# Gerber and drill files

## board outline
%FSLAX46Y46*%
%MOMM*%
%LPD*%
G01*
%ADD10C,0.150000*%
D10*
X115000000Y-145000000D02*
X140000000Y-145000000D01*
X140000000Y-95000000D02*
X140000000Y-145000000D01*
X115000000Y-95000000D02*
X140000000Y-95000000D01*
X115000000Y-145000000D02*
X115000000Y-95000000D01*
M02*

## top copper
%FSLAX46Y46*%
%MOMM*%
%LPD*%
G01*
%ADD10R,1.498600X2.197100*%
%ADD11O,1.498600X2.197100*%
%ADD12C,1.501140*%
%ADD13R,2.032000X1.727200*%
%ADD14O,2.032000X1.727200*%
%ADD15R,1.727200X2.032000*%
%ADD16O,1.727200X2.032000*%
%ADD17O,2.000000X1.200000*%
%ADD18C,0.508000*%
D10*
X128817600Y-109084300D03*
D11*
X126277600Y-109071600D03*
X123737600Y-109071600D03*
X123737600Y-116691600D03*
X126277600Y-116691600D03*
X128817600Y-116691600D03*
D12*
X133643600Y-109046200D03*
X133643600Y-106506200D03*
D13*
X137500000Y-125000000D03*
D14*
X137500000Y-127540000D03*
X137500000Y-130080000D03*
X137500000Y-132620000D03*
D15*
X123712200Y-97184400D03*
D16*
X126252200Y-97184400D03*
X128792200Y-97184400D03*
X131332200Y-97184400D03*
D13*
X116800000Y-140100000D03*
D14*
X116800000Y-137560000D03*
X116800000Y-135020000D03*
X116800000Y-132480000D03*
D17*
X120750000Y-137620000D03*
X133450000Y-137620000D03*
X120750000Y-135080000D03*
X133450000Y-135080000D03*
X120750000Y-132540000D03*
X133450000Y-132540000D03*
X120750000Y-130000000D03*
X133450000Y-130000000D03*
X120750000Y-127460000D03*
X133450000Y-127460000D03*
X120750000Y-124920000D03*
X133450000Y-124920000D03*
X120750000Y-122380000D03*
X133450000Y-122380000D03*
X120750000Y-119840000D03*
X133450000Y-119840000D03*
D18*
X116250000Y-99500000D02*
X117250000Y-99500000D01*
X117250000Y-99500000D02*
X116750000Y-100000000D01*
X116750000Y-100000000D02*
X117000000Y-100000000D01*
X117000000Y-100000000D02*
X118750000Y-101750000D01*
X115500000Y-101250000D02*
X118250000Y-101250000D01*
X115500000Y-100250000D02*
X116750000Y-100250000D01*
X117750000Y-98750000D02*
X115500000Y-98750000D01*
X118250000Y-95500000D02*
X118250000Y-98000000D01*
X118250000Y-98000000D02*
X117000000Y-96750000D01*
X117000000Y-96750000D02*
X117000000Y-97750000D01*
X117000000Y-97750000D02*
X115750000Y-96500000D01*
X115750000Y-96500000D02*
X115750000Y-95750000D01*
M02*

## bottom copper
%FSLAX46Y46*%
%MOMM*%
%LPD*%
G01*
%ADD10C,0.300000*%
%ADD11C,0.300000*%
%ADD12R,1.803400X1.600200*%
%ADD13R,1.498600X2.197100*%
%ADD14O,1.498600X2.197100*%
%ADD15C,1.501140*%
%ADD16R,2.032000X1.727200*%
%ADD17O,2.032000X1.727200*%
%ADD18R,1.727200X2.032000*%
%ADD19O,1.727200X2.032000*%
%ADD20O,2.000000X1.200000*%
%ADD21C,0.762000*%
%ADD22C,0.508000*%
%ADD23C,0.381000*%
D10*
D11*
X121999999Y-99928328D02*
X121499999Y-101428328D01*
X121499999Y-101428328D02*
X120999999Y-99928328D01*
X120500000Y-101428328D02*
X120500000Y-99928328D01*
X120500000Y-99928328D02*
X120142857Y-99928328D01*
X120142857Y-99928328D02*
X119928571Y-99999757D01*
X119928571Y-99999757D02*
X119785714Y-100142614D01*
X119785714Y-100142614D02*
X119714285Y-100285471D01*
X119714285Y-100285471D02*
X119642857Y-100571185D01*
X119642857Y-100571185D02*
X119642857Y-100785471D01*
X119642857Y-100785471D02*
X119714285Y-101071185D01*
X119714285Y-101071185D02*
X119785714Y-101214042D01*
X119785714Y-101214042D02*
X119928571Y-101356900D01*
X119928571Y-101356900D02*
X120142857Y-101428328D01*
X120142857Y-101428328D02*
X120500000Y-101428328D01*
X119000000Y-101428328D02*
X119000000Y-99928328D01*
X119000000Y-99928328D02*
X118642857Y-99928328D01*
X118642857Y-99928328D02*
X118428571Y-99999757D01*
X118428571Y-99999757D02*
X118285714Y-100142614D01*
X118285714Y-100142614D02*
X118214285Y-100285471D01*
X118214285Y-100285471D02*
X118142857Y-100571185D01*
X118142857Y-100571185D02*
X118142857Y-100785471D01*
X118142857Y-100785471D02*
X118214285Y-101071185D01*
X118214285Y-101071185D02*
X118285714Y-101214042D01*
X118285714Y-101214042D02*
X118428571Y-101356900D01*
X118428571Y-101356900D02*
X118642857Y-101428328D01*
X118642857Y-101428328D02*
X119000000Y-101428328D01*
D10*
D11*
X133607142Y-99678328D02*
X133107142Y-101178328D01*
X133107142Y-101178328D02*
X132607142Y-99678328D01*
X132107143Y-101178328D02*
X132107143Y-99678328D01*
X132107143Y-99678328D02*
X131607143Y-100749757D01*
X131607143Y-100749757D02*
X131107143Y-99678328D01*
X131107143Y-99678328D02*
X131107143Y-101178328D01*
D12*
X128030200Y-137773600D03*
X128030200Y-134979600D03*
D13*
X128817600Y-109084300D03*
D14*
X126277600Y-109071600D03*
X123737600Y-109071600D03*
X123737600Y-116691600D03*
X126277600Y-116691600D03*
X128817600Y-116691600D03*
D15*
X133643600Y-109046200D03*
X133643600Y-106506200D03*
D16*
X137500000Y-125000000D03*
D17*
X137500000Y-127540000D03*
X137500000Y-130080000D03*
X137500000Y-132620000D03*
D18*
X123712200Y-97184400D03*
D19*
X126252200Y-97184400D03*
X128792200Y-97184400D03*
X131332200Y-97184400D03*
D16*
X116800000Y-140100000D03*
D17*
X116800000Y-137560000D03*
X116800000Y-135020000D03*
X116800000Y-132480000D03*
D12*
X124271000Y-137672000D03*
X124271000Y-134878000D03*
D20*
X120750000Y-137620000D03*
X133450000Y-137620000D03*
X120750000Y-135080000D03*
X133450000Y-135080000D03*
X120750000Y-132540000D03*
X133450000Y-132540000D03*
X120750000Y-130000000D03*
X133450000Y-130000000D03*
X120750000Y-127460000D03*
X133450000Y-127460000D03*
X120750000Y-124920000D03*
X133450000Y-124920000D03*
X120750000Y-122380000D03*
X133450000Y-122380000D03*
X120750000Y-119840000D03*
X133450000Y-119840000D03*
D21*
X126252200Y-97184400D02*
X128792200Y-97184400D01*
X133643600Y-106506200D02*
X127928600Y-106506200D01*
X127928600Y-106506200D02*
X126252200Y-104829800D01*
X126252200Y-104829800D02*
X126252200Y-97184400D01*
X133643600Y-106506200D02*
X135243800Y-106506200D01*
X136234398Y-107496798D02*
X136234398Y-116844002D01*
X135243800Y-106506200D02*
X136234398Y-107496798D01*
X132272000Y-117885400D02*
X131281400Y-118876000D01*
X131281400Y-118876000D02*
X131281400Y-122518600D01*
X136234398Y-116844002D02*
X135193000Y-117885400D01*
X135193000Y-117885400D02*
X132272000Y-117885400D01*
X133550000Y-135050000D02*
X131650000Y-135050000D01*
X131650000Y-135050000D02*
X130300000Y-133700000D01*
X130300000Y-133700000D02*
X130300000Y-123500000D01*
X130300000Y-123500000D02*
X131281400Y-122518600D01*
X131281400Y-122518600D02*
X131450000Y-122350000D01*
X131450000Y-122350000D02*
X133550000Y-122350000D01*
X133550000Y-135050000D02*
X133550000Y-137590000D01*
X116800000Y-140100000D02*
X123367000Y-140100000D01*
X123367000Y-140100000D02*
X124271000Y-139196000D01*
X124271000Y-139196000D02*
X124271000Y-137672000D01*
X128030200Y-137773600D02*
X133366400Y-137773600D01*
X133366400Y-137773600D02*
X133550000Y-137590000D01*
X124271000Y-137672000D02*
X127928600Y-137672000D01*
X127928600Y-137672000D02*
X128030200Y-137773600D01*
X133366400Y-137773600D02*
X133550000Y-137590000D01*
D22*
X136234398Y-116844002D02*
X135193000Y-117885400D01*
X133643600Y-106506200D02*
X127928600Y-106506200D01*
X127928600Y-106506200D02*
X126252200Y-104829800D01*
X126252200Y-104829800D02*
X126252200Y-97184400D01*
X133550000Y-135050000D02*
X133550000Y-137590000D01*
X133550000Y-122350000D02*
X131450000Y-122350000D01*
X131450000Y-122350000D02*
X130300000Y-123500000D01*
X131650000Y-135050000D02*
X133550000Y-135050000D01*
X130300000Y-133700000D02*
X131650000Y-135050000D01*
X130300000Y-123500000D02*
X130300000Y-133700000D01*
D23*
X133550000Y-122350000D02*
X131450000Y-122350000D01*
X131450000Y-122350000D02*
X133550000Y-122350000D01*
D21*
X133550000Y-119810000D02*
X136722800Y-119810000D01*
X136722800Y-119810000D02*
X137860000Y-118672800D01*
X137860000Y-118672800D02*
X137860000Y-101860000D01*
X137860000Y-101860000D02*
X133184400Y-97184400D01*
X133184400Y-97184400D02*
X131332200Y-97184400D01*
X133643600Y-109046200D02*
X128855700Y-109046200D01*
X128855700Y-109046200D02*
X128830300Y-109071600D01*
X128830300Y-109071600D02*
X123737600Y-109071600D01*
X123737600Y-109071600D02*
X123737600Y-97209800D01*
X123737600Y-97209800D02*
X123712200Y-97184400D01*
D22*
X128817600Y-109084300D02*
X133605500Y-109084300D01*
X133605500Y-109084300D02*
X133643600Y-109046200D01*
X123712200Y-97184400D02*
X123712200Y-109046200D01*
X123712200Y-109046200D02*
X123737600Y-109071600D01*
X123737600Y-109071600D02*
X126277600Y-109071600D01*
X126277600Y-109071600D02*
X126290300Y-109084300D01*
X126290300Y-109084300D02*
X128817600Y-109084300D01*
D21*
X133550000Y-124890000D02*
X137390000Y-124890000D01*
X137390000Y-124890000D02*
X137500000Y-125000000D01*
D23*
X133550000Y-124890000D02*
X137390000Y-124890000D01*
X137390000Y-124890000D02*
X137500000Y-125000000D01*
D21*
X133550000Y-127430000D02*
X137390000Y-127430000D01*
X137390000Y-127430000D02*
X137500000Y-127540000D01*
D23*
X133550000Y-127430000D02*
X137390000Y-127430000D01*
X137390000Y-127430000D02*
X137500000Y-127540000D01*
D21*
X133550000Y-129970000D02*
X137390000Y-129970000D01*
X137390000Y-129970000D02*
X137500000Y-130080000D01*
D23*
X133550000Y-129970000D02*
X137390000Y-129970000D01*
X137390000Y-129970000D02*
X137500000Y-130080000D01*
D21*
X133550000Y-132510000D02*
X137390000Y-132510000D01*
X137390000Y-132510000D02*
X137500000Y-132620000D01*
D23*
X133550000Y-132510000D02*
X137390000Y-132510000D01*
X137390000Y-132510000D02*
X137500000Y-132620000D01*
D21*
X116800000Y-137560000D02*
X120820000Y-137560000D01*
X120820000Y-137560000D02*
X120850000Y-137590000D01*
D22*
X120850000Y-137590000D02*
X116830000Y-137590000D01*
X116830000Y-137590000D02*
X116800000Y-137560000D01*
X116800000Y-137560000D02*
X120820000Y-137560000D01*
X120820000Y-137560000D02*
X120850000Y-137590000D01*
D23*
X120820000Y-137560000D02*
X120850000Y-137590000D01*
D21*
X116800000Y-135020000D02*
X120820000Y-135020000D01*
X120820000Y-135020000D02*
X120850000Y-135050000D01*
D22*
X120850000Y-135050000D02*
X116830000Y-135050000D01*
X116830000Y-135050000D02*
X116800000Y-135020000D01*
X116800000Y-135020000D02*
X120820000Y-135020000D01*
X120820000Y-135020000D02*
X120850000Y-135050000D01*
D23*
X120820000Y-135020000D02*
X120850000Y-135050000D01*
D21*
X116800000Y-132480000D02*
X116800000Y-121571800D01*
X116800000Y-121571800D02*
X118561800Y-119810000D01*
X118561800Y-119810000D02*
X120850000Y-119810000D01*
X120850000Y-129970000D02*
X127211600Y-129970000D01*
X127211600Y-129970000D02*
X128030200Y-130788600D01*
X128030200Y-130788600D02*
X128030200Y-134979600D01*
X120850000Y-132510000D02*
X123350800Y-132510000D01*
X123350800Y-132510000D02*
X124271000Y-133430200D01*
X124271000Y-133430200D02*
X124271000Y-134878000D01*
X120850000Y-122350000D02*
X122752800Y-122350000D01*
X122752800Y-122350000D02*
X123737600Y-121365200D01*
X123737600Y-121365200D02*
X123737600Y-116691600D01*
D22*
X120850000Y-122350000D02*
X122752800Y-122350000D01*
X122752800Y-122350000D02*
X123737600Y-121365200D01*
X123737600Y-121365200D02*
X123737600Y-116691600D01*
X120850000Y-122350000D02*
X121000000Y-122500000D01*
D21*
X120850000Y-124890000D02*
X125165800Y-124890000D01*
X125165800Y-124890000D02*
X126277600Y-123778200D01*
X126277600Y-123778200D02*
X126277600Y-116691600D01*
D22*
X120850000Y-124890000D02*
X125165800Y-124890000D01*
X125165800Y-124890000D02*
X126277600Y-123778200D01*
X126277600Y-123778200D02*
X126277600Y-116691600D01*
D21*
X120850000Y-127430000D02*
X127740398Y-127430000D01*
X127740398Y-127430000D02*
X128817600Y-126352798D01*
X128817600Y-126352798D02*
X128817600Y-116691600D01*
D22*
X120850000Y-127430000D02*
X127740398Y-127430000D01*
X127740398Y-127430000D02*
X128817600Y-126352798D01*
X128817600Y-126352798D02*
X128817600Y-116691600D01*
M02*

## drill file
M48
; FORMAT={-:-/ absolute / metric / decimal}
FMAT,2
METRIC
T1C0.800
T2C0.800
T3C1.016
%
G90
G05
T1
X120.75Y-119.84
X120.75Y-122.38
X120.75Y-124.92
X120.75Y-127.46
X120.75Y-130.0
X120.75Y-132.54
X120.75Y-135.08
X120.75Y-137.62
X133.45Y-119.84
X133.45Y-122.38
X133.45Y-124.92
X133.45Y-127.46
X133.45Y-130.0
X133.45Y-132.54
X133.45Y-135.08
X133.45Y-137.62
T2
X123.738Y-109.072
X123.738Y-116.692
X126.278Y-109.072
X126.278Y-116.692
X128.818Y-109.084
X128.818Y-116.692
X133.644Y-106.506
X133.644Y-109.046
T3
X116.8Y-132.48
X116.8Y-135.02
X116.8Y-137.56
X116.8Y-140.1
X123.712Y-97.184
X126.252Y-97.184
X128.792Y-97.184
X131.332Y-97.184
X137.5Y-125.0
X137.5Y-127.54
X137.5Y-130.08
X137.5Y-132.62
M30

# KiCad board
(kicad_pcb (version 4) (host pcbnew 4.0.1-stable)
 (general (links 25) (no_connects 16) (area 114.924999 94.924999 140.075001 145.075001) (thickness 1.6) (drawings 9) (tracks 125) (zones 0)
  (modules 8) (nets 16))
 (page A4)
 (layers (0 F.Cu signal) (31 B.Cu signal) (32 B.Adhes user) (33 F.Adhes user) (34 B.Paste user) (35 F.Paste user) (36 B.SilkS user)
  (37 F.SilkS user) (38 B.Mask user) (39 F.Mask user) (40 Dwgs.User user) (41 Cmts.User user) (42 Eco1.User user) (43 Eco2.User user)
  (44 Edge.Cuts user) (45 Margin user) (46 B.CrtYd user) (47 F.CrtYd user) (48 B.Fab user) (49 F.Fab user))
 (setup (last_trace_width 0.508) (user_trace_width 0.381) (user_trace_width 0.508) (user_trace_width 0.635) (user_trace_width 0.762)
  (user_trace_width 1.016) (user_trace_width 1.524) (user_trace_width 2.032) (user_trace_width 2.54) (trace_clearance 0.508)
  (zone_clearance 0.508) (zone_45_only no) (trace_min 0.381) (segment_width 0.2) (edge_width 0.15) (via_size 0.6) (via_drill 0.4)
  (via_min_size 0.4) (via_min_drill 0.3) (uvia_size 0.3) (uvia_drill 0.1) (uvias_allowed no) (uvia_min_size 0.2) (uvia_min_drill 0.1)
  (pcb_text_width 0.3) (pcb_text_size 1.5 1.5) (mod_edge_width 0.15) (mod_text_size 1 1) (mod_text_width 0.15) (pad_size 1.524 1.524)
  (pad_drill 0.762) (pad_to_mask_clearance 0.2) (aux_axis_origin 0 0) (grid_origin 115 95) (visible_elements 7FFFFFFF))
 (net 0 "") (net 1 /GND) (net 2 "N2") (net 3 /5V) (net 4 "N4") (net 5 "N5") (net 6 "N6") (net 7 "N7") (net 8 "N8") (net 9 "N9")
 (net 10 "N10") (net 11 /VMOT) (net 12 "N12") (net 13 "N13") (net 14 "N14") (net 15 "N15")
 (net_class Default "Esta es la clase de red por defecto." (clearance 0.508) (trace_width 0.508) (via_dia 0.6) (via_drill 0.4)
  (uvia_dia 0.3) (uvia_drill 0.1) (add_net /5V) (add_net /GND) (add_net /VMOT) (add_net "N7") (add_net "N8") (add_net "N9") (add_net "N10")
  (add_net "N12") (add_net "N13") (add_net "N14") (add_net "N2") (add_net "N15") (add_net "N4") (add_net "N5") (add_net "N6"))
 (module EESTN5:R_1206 (layer B.Cu) (at 128.0302 136.3766 270)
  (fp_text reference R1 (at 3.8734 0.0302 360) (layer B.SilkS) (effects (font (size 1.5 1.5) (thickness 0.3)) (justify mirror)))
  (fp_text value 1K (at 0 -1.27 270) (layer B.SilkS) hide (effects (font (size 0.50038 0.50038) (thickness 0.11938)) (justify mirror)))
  (pad 1 smd rect (at 1.397 0 270) (size 1.6002 1.8034) (layers B.Cu B.Paste B.Mask) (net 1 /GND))
  (pad 2 smd rect (at -1.397 0 270) (size 1.6002 1.8034) (layers B.Cu B.Paste B.Mask) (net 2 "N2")))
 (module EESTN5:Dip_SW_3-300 (layer F.Cu) (at 126.2776 112.8816 180)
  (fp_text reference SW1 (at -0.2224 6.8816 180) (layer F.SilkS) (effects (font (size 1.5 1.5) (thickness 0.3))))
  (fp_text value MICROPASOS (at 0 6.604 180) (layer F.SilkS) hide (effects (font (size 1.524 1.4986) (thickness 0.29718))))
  (pad 1 thru_hole rect (at -2.54 3.7973 180) (size 1.4986 2.1971) (drill 0.8001) (layers *.Cu *.Mask F.SilkS) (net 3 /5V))
  (pad 2 thru_hole oval (at 0 3.81 180) (size 1.4986 2.1971) (drill 0.8001) (layers *.Cu *.Mask F.SilkS) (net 3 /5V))
  (pad 3 thru_hole oval (at 2.54 3.81 180) (size 1.4986 2.1971) (drill 0.8001) (layers *.Cu *.Mask F.SilkS) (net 3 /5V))
  (pad 4 thru_hole oval (at 2.54 -3.81 180) (size 1.4986 2.1971) (drill 0.8001) (layers *.Cu *.Mask F.SilkS) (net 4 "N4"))
  (pad 5 thru_hole oval (at 0 -3.81 180) (size 1.4986 2.1971) (drill 0.8001) (layers *.Cu *.Mask F.SilkS) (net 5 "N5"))
  (pad 6 thru_hole oval (at -2.54 -3.81 180) (size 1.4986 2.1971) (drill 0.8001) (layers *.Cu *.Mask F.SilkS) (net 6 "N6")))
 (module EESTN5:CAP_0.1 (layer F.Cu) (at 133.6436 107.7762 90)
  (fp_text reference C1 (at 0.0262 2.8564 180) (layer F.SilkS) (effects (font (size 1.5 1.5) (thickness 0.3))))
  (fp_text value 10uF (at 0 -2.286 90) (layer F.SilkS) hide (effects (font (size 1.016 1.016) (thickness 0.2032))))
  (pad 1 thru_hole circle (at -1.27 0 90) (size 1.50114 1.50114) (drill 0.8001) (layers *.Cu *.Mask F.SilkS) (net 3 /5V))
  (pad 2 thru_hole circle (at 1.27 0 90) (size 1.50114 1.50114) (drill 0.8001) (layers *.Cu *.Mask F.SilkS) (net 1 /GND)))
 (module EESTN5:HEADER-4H (layer F.Cu) (at 137.5 125)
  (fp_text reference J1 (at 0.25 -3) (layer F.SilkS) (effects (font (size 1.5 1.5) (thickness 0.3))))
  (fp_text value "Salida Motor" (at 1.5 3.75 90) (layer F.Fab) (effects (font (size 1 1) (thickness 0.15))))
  (pad 1 thru_hole rect (at 0 0) (size 2.032 1.7272) (drill 1.016) (layers *.Cu *.Mask F.SilkS) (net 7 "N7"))
  (pad 2 thru_hole oval (at 0 2.54) (size 2.032 1.7272) (drill 1.016) (layers *.Cu *.Mask F.SilkS) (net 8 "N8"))
  (pad 3 thru_hole oval (at 0 5.08) (size 2.032 1.7272) (drill 1.016) (layers *.Cu *.Mask F.SilkS) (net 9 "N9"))
  (pad 4 thru_hole oval (at 0 7.62) (size 2.032 1.7272) (drill 1.016) (layers *.Cu *.Mask F.SilkS) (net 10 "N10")))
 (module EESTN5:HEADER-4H (layer F.Cu) (at 123.7122 97.1844 90)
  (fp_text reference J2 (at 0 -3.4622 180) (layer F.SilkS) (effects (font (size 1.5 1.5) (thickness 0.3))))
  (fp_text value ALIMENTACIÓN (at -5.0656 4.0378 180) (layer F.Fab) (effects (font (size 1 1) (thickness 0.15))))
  (pad 1 thru_hole rect (at 0 0 90) (size 2.032 1.7272) (drill 1.016) (layers *.Cu *.Mask F.SilkS) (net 3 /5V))
  (pad 2 thru_hole oval (at 0 2.54 90) (size 2.032 1.7272) (drill 1.016) (layers *.Cu *.Mask F.SilkS) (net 1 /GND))
  (pad 3 thru_hole oval (at 0 5.08 90) (size 2.032 1.7272) (drill 1.016) (layers *.Cu *.Mask F.SilkS) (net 1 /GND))
  (pad 4 thru_hole oval (at 0 7.62 90) (size 2.032 1.7272) (drill 1.016) (layers *.Cu *.Mask F.SilkS) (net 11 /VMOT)))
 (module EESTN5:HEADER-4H (layer F.Cu) (at 116.8 140.1 180)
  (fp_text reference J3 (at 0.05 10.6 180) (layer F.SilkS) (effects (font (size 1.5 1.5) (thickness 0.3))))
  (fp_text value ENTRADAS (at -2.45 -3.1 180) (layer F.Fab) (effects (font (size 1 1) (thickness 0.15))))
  (pad 1 thru_hole rect (at 0 0 180) (size 2.032 1.7272) (drill 1.016) (layers *.Cu *.Mask F.SilkS) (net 1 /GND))
  (pad 2 thru_hole oval (at 0 2.54 180) (size 2.032 1.7272) (drill 1.016) (layers *.Cu *.Mask F.SilkS) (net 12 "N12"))
  (pad 3 thru_hole oval (at 0 5.08 180) (size 2.032 1.7272) (drill 1.016) (layers *.Cu *.Mask F.SilkS) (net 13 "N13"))
  (pad 4 thru_hole oval (at 0 7.62 180) (size 2.032 1.7272) (drill 1.016) (layers *.Cu *.Mask F.SilkS) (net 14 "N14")))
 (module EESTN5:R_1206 (layer B.Cu) (at 124.271 136.275 270)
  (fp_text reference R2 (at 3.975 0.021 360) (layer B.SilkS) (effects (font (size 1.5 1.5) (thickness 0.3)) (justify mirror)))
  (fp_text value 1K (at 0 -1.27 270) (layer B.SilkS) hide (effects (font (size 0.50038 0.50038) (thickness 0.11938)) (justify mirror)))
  (pad 1 smd rect (at 1.397 0 270) (size 1.6002 1.8034) (layers B.Cu B.Paste B.Mask) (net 1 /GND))
  (pad 2 smd rect (at -1.397 0 270) (size 1.6002 1.8034) (layers B.Cu B.Paste B.Mask) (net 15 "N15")))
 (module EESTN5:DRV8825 (layer F.Cu) (at 127.1 128.73 90)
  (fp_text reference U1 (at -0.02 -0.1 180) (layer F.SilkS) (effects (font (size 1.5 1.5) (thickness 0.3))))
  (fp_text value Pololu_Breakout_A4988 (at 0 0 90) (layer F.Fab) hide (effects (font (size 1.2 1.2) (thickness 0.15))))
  (pad 16 thru_hole oval (at -8.89 -6.35 90) (size 1.2 2) (drill 0.8) (layers *.Cu *.Mask F.SilkS) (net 12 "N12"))
  (pad 1 thru_hole oval (at -8.89 6.35 90) (size 1.2 2) (drill 0.8) (layers *.Cu *.Mask F.SilkS) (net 1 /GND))
  (pad 15 thru_hole oval (at -6.35 -6.35 90) (size 1.2 2) (drill 0.8) (layers *.Cu *.Mask F.SilkS) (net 13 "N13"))
  (pad 2 thru_hole oval (at -6.35 6.35 90) (size 1.2 2) (drill 0.8) (layers *.Cu *.Mask F.SilkS) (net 1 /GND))
  (pad 14 thru_hole oval (at -3.81 -6.35 90) (size 1.2 2) (drill 0.8) (layers *.Cu *.Mask F.SilkS) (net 15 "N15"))
  (pad 3 thru_hole oval (at -3.81 6.35 90) (size 1.2 2) (drill 0.8) (layers *.Cu *.Mask F.SilkS) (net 10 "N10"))
  (pad 13 thru_hole oval (at -1.27 -6.35 90) (size 1.2 2) (drill 0.8) (layers *.Cu *.Mask F.SilkS) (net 2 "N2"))
  (pad 4 thru_hole oval (at -1.27 6.35 90) (size 1.2 2) (drill 0.8) (layers *.Cu *.Mask F.SilkS) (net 9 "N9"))
  (pad 12 thru_hole oval (at 1.27 -6.35 90) (size 1.2 2) (drill 0.8) (layers *.Cu *.Mask F.SilkS) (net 6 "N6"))
  (pad 5 thru_hole oval (at 1.27 6.35 90) (size 1.2 2) (drill 0.8) (layers *.Cu *.Mask F.SilkS) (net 8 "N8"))
  (pad 11 thru_hole oval (at 3.81 -6.35 90) (size 1.2 2) (drill 0.8) (layers *.Cu *.Mask F.SilkS) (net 5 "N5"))
  (pad 6 thru_hole oval (at 3.81 6.35 90) (size 1.2 2) (drill 0.8) (layers *.Cu *.Mask F.SilkS) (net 7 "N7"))
  (pad 10 thru_hole oval (at 6.35 -6.35 90) (size 1.2 2) (drill 0.8) (layers *.Cu *.Mask F.SilkS) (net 4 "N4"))
  (pad 7 thru_hole oval (at 6.35 6.35 90) (size 1.2 2) (drill 0.8) (layers *.Cu *.Mask F.SilkS) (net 1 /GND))
  (pad 9 thru_hole oval (at 8.89 -6.35 90) (size 1.2 2) (drill 0.8) (layers *.Cu *.Mask F.SilkS) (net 14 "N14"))
  (pad 8 thru_hole oval (at 8.89 6.35 90) (size 1.2 2) (drill 0.8) (layers *.Cu *.Mask F.SilkS) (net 11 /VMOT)))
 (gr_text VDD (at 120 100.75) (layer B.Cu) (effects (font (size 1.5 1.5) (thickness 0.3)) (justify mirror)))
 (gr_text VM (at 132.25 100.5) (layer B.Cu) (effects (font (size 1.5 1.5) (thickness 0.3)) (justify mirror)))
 (gr_line (start 115 145) (end 140 145) (angle 90) (layer Edge.Cuts) (width 0.15))
 (gr_line (start 140 95) (end 140 145) (angle 90) (layer Edge.Cuts) (width 0.15))
 (gr_line (start 115 95) (end 140 95) (angle 90) (layer Edge.Cuts) (width 0.15))
 (gr_line (start 115 145) (end 115 95) (angle 90) (layer Edge.Cuts) (width 0.15))
 (segment (start 116.25 99.5) (end 117.25 99.5) (width 0.508) (layer F.Cu) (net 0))
 (segment (start 117.25 99.5) (end 116.75 100) (width 0.508) (layer F.Cu) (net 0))
 (segment (start 116.75 100) (end 117 100) (width 0.508) (layer F.Cu) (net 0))
 (segment (start 117 100) (end 118.75 101.75) (width 0.508) (layer F.Cu) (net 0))
 (segment (start 115.5 101.25) (end 118.25 101.25) (width 0.508) (layer F.Cu) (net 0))
 (segment (start 115.5 100.25) (end 116.75 100.25) (width 0.508) (layer F.Cu) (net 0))
 (segment (start 117.75 98.75) (end 115.5 98.75) (width 0.508) (layer F.Cu) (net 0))
 (segment (start 118.25 95.5) (end 118.25 98) (width 0.508) (layer F.Cu) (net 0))
 (segment (start 118.25 98) (end 117 96.75) (width 0.508) (layer F.Cu) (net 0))
 (segment (start 117 96.75) (end 117 97.75) (width 0.508) (layer F.Cu) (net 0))
 (segment (start 117 97.75) (end 115.75 96.5) (width 0.508) (layer F.Cu) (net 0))
 (segment (start 115.75 96.5) (end 115.75 95.75) (width 0.508) (layer F.Cu) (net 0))
 (segment (start 126.2522 97.1844) (end 128.7922 97.1844) (width 0.762) (layer B.Cu) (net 1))
 (segment (start 133.6436 106.5062) (end 127.9286 106.5062) (width 0.762) (layer B.Cu) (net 1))
 (segment (start 127.9286 106.5062) (end 126.2522 104.8298) (width 0.762) (layer B.Cu) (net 1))
 (segment (start 126.2522 104.8298) (end 126.2522 97.1844) (width 0.762) (layer B.Cu) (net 1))
 (segment (start 133.6436 106.5062) (end 135.2438 106.5062) (width 0.762) (layer B.Cu) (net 1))
 (segment (start 136.234398 107.496798) (end 136.234398 116.844002) (width 0.762) (layer B.Cu) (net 1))
 (segment (start 135.2438 106.5062) (end 136.234398 107.496798) (width 0.762) (layer B.Cu) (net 1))
 (segment (start 132.272 117.8854) (end 131.2814 118.876) (width 0.762) (layer B.Cu) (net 1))
 (segment (start 131.2814 118.876) (end 131.2814 122.5186) (width 0.762) (layer B.Cu) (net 1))
 (segment (start 136.234398 116.844002) (end 135.193 117.8854) (width 0.762) (layer B.Cu) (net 1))
 (segment (start 135.193 117.8854) (end 132.272 117.8854) (width 0.762) (layer B.Cu) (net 1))
 (segment (start 133.55 135.05) (end 131.65 135.05) (width 0.762) (layer B.Cu) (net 1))
 (segment (start 131.65 135.05) (end 130.3 133.7) (width 0.762) (layer B.Cu) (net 1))
 (segment (start 130.3 133.7) (end 130.3 123.5) (width 0.762) (layer B.Cu) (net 1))
 (segment (start 130.3 123.5) (end 131.2814 122.5186) (width 0.762) (layer B.Cu) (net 1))
 (segment (start 131.2814 122.5186) (end 131.45 122.35) (width 0.762) (layer B.Cu) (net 1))
 (segment (start 131.45 122.35) (end 133.55 122.35) (width 0.762) (layer B.Cu) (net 1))
 (segment (start 133.55 135.05) (end 133.55 137.59) (width 0.762) (layer B.Cu) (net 1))
 (segment (start 116.8 140.1) (end 123.367 140.1) (width 0.762) (layer B.Cu) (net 1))
 (segment (start 123.367 140.1) (end 124.271 139.196) (width 0.762) (layer B.Cu) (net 1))
 (segment (start 124.271 139.196) (end 124.271 137.672) (width 0.762) (layer B.Cu) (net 1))
 (segment (start 128.0302 137.7736) (end 133.3664 137.7736) (width 0.762) (layer B.Cu) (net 1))
 (segment (start 133.3664 137.7736) (end 133.55 137.59) (width 0.762) (layer B.Cu) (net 1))
 (segment (start 124.271 137.672) (end 127.9286 137.672) (width 0.762) (layer B.Cu) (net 1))
 (segment (start 127.9286 137.672) (end 128.0302 137.7736) (width 0.762) (layer B.Cu) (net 1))
 (segment (start 133.3664 137.7736) (end 133.55 137.59) (width 0.762) (layer B.Cu) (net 1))
 (segment (start 136.234398 116.844002) (end 135.193 117.8854) (width 0.508) (layer B.Cu) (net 1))
 (segment (start 133.6436 106.5062) (end 127.9286 106.5062) (width 0.508) (layer B.Cu) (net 1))
 (segment (start 127.9286 106.5062) (end 126.2522 104.8298) (width 0.508) (layer B.Cu) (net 1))
 (segment (start 126.2522 104.8298) (end 126.2522 97.1844) (width 0.508) (layer B.Cu) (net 1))
 (segment (start 133.55 135.05) (end 133.55 137.59) (width 0.508) (layer B.Cu) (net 1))
 (segment (start 133.55 122.35) (end 131.45 122.35) (width 0.508) (layer B.Cu) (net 1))
 (segment (start 131.45 122.35) (end 130.3 123.5) (width 0.508) (layer B.Cu) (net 1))
 (segment (start 131.65 135.05) (end 133.55 135.05) (width 0.508) (layer B.Cu) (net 1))
 (segment (start 130.3 133.7) (end 131.65 135.05) (width 0.508) (layer B.Cu) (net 1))
 (segment (start 130.3 123.5) (end 130.3 133.7) (width 0.508) (layer B.Cu) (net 1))
 (segment (start 133.55 122.35) (end 131.45 122.35) (width 0.381) (layer B.Cu) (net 1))
 (segment (start 131.45 122.35) (end 133.55 122.35) (width 0.381) (layer B.Cu) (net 1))
 (segment (start 133.55 119.81) (end 136.7228 119.81) (width 0.762) (layer B.Cu) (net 11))
 (segment (start 136.7228 119.81) (end 137.86 118.6728) (width 0.762) (layer B.Cu) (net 11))
 (segment (start 137.86 118.6728) (end 137.86 101.86) (width 0.762) (layer B.Cu) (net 11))
 (segment (start 137.86 101.86) (end 133.1844 97.1844) (width 0.762) (layer B.Cu) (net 11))
 (segment (start 133.1844 97.1844) (end 131.3322 97.1844) (width 0.762) (layer B.Cu) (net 11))
 (segment (start 133.6436 109.0462) (end 128.8557 109.0462) (width 0.762) (layer B.Cu) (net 3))
 (segment (start 128.8557 109.0462) (end 128.8303 109.0716) (width 0.762) (layer B.Cu) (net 3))
 (segment (start 128.8303 109.0716) (end 123.7376 109.0716) (width 0.762) (layer B.Cu) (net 3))
 (segment (start 123.7376 109.0716) (end 123.7376 97.2098) (width 0.762) (layer B.Cu) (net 3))
 (segment (start 123.7376 97.2098) (end 123.7122 97.1844) (width 0.762) (layer B.Cu) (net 3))
 (segment (start 128.8176 109.0843) (end 133.6055 109.0843) (width 0.508) (layer B.Cu) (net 3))
 (segment (start 133.6055 109.0843) (end 133.6436 109.0462) (width 0.508) (layer B.Cu) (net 3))
 (segment (start 123.7122 97.1844) (end 123.7122 109.0462) (width 0.508) (layer B.Cu) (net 3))
 (segment (start 123.7122 109.0462) (end 123.7376 109.0716) (width 0.508) (layer B.Cu) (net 3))
 (segment (start 123.7376 109.0716) (end 126.2776 109.0716) (width 0.508) (layer B.Cu) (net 3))
 (segment (start 126.2776 109.0716) (end 126.2903 109.0843) (width 0.508) (layer B.Cu) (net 3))
 (segment (start 126.2903 109.0843) (end 128.8176 109.0843) (width 0.508) (layer B.Cu) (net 3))
 (segment (start 133.55 124.89) (end 137.39 124.89) (width 0.762) (layer B.Cu) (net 7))
 (segment (start 137.39 124.89) (end 137.5 125) (width 0.762) (layer B.Cu) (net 7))
 (segment (start 133.55 124.89) (end 137.39 124.89) (width 0.381) (layer B.Cu) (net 7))
 (segment (start 137.39 124.89) (end 137.5 125) (width 0.381) (layer B.Cu) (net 7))
 (segment (start 133.55 127.43) (end 137.39 127.43) (width 0.762) (layer B.Cu) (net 8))
 (segment (start 137.39 127.43) (end 137.5 127.54) (width 0.762) (layer B.Cu) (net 8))
 (segment (start 133.55 127.43) (end 137.39 127.43) (width 0.381) (layer B.Cu) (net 8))
 (segment (start 137.39 127.43) (end 137.5 127.54) (width 0.381) (layer B.Cu) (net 8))
 (segment (start 133.55 129.97) (end 137.39 129.97) (width 0.762) (layer B.Cu) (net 9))
 (segment (start 137.39 129.97) (end 137.5 130.08) (width 0.762) (layer B.Cu) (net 9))
 (segment (start 133.55 129.97) (end 137.39 129.97) (width 0.381) (layer B.Cu) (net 9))
 (segment (start 137.39 129.97) (end 137.5 130.08) (width 0.381) (layer B.Cu) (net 9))
 (segment (start 133.55 132.51) (end 137.39 132.51) (width 0.762) (layer B.Cu) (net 10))
 (segment (start 137.39 132.51) (end 137.5 132.62) (width 0.762) (layer B.Cu) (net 10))
 (segment (start 133.55 132.51) (end 137.39 132.51) (width 0.381) (layer B.Cu) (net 10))
 (segment (start 137.39 132.51) (end 137.5 132.62) (width 0.381) (layer B.Cu) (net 10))
 (segment (start 116.8 137.56) (end 120.82 137.56) (width 0.762) (layer B.Cu) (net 12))
 (segment (start 120.82 137.56) (end 120.85 137.59) (width 0.762) (layer B.Cu) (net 12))
 (segment (start 120.85 137.59) (end 116.83 137.59) (width 0.508) (layer B.Cu) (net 12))
 (segment (start 116.83 137.59) (end 116.8 137.56) (width 0.508) (layer B.Cu) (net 12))
 (segment (start 116.8 137.56) (end 120.82 137.56) (width 0.508) (layer B.Cu) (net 12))
 (segment (start 120.82 137.56) (end 120.85 137.59) (width 0.508) (layer B.Cu) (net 12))
 (segment (start 120.82 137.56) (end 120.85 137.59) (width 0.381) (layer B.Cu) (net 12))
 (segment (start 116.8 135.02) (end 120.82 135.02) (width 0.762) (layer B.Cu) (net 13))
 (segment (start 120.82 135.02) (end 120.85 135.05) (width 0.762) (layer B.Cu) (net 13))
 (segment (start 120.85 135.05) (end 116.83 135.05) (width 0.508) (layer B.Cu) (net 13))
 (segment (start 116.83 135.05) (end 116.8 135.02) (width 0.508) (layer B.Cu) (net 13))
 (segment (start 116.8 135.02) (end 120.82 135.02) (width 0.508) (layer B.Cu) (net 13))
 (segment (start 120.82 135.02) (end 120.85 135.05) (width 0.508) (layer B.Cu) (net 13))
 (segment (start 120.82 135.02) (end 120.85 135.05) (width 0.381) (layer B.Cu) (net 13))
 (segment (start 116.8 132.48) (end 116.8 121.5718) (width 0.762) (layer B.Cu) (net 14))
 (segment (start 116.8 121.5718) (end 118.5618 119.81) (width 0.762) (layer B.Cu) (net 14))
 (segment (start 118.5618 119.81) (end 120.85 119.81) (width 0.762) (layer B.Cu) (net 14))
 (segment (start 120.85 129.97) (end 127.2116 129.97) (width 0.762) (layer B.Cu) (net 2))
 (segment (start 127.2116 129.97) (end 128.0302 130.7886) (width 0.762) (layer B.Cu) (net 2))
 (segment (start 128.0302 130.7886) (end 128.0302 134.9796) (width 0.762) (layer B.Cu) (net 2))
 (segment (start 120.85 132.51) (end 123.3508 132.51) (width 0.762) (layer B.Cu) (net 15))
 (segment (start 123.3508 132.51) (end 124.271 133.4302) (width 0.762) (layer B.Cu) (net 15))
 (segment (start 124.271 133.4302) (end 124.271 134.878) (width 0.762) (layer B.Cu) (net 15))
 (segment (start 120.85 122.35) (end 122.7528 122.35) (width 0.762) (layer B.Cu) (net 4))
 (segment (start 122.7528 122.35) (end 123.7376 121.3652) (width 0.762) (layer B.Cu) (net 4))
 (segment (start 123.7376 121.3652) (end 123.7376 116.6916) (width 0.762) (layer B.Cu) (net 4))
 (segment (start 120.85 122.35) (end 122.7528 122.35) (width 0.508) (layer B.Cu) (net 4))
 (segment (start 122.7528 122.35) (end 123.7376 121.3652) (width 0.508) (layer B.Cu) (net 4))
 (segment (start 123.7376 121.3652) (end 123.7376 116.6916) (width 0.508) (layer B.Cu) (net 4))
 (segment (start 120.85 122.35) (end 121 122.5) (width 0.508) (layer B.Cu) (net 4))
 (segment (start 120.85 124.89) (end 125.1658 124.89) (width 0.762) (layer B.Cu) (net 5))
 (segment (start 125.1658 124.89) (end 126.2776 123.7782) (width 0.762) (layer B.Cu) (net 5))
 (segment (start 126.2776 123.7782) (end 126.2776 116.6916) (width 0.762) (layer B.Cu) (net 5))
 (segment (start 120.85 124.89) (end 125.1658 124.89) (width 0.508) (layer B.Cu) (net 5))
 (segment (start 125.1658 124.89) (end 126.2776 123.7782) (width 0.508) (layer B.Cu) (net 5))
 (segment (start 126.2776 123.7782) (end 126.2776 116.6916) (width 0.508) (layer B.Cu) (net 5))
 (segment (start 120.85 127.43) (end 127.740398 127.43) (width 0.762) (layer B.Cu) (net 6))
 (segment (start 127.740398 127.43) (end 128.8176 126.352798) (width 0.762) (layer B.Cu) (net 6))
 (segment (start 128.8176 126.352798) (end 128.8176 116.6916) (width 0.762) (layer B.Cu) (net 6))
 (segment (start 120.85 127.43) (end 127.740398 127.43) (width 0.508) (layer B.Cu) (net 6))
 (segment (start 127.740398 127.43) (end 128.8176 126.352798) (width 0.508) (layer B.Cu) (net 6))
 (segment (start 128.8176 126.352798) (end 128.8176 116.6916) (width 0.508) (layer B.Cu) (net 6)))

